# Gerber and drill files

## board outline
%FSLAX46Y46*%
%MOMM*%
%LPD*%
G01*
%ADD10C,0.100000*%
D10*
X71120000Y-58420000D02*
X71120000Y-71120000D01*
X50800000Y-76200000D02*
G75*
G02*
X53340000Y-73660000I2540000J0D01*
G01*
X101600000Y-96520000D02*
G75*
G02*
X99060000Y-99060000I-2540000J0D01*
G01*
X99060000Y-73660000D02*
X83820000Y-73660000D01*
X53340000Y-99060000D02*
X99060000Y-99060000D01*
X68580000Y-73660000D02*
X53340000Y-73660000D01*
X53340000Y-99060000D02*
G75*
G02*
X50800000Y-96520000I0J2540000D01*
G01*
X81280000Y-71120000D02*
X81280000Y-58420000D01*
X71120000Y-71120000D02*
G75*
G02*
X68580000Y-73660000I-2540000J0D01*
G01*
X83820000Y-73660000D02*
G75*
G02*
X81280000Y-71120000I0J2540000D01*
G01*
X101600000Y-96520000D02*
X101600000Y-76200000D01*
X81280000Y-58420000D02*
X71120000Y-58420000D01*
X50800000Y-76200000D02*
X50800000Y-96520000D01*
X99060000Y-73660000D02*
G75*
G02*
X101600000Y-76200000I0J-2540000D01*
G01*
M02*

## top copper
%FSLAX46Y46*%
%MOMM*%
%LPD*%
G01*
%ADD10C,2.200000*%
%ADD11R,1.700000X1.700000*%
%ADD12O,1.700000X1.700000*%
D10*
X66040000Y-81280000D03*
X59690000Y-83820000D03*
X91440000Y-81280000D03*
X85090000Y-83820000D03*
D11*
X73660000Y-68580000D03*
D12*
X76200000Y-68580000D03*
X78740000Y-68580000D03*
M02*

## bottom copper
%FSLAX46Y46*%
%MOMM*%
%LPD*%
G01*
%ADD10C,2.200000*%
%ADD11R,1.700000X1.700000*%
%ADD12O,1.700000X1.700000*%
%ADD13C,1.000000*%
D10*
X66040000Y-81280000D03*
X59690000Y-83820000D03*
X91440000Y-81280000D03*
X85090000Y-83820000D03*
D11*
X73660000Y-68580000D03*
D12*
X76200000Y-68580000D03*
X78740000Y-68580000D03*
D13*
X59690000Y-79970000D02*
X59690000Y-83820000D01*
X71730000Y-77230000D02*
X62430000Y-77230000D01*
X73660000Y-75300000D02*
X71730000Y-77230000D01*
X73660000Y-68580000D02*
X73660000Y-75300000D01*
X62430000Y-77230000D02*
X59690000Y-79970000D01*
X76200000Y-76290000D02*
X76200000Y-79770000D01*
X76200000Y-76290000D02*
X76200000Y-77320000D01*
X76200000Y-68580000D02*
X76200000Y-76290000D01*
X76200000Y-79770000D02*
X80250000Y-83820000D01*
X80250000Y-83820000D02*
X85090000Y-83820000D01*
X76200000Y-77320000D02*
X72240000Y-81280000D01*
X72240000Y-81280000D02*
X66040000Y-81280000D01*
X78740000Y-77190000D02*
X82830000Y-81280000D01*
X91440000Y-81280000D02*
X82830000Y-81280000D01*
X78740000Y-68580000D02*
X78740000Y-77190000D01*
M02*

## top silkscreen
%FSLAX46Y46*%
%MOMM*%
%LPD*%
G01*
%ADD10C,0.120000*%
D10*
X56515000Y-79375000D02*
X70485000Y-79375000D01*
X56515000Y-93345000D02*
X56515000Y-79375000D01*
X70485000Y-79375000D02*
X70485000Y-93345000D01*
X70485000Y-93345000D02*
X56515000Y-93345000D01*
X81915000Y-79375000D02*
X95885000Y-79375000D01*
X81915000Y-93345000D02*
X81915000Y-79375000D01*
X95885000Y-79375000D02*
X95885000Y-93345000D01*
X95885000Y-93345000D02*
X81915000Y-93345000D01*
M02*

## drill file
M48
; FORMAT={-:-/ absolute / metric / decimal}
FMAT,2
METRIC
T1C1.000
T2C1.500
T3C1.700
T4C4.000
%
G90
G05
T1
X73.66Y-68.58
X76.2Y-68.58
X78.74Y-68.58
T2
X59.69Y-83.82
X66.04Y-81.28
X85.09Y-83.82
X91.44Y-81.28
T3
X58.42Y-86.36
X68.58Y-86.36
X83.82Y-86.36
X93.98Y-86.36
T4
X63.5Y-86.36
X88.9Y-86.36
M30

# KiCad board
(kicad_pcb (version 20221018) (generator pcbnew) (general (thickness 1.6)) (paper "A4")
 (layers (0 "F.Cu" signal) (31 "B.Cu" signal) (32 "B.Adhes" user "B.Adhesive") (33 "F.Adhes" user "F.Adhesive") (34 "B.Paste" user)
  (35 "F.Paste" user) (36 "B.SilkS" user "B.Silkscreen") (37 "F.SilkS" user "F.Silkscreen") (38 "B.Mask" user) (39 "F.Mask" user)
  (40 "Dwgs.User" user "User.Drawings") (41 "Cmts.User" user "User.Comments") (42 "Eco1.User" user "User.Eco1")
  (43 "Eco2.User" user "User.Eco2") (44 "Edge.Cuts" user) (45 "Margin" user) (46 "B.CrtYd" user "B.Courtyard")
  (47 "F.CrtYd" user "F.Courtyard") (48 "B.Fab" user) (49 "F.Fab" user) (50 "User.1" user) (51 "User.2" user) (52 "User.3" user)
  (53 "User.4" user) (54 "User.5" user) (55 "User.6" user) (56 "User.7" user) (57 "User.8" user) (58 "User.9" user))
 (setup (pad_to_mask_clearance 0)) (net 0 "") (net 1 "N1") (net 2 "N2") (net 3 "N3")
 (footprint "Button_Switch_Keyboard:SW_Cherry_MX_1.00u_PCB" (layer "F.Cu") (at 66.04 81.28)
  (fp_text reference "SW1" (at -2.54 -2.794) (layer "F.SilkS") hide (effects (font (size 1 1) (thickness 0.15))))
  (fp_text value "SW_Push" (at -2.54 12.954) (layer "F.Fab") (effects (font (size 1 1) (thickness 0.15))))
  (fp_line (start -9.525 -1.905) (end 4.445 -1.905) (stroke (width 0.12) (type solid)) (layer "F.SilkS"))
  (fp_line (start -9.525 12.065) (end -9.525 -1.905) (stroke (width 0.12) (type solid)) (layer "F.SilkS"))
  (fp_line (start 4.445 -1.905) (end 4.445 12.065) (stroke (width 0.12) (type solid)) (layer "F.SilkS"))
  (fp_line (start 4.445 12.065) (end -9.525 12.065) (stroke (width 0.12) (type solid)) (layer "F.SilkS"))
  (pad "" np_thru_hole circle (at -7.62 5.08) (size 1.7 1.7) (drill 1.7) (layers "*.Cu" "*.Mask"))
  (pad "" np_thru_hole circle (at -2.54 5.08) (size 4 4) (drill 4) (layers "*.Cu" "*.Mask"))
  (pad "" np_thru_hole circle (at 2.54 5.08) (size 1.7 1.7) (drill 1.7) (layers "*.Cu" "*.Mask"))
  (pad "1" thru_hole circle (at 0 0) (size 2.2 2.2) (drill 1.5) (layers "*.Cu" "*.Mask") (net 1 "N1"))
  (pad "2" thru_hole circle (at -6.35 2.54) (size 2.2 2.2) (drill 1.5) (layers "*.Cu" "*.Mask") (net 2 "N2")))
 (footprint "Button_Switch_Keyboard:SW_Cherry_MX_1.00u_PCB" (layer "F.Cu") (at 91.44 81.28)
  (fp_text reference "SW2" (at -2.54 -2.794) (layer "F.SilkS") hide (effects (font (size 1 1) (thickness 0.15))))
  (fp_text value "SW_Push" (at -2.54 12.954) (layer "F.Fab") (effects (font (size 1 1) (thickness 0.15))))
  (fp_line (start -9.525 -1.905) (end 4.445 -1.905) (stroke (width 0.12) (type solid)) (layer "F.SilkS"))
  (fp_line (start -9.525 12.065) (end -9.525 -1.905) (stroke (width 0.12) (type solid)) (layer "F.SilkS"))
  (fp_line (start 4.445 -1.905) (end 4.445 12.065) (stroke (width 0.12) (type solid)) (layer "F.SilkS"))
  (fp_line (start 4.445 12.065) (end -9.525 12.065) (stroke (width 0.12) (type solid)) (layer "F.SilkS"))
  (pad "" np_thru_hole circle (at -7.62 5.08) (size 1.7 1.7) (drill 1.7) (layers "*.Cu" "*.Mask"))
  (pad "" np_thru_hole circle (at -2.54 5.08) (size 4 4) (drill 4) (layers "*.Cu" "*.Mask"))
  (pad "" np_thru_hole circle (at 2.54 5.08) (size 1.7 1.7) (drill 1.7) (layers "*.Cu" "*.Mask"))
  (pad "1" thru_hole circle (at 0 0) (size 2.2 2.2) (drill 1.5) (layers "*.Cu" "*.Mask") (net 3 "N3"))
  (pad "2" thru_hole circle (at -6.35 2.54) (size 2.2 2.2) (drill 1.5) (layers "*.Cu" "*.Mask") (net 1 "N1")))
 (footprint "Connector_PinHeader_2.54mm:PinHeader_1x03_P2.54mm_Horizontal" (layer "F.Cu") (at 73.66 68.58 90)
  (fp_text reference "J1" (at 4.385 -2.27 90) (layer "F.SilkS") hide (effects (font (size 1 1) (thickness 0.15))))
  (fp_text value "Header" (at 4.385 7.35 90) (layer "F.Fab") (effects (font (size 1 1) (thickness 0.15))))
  (pad "1" thru_hole rect (at 0 0 90) (size 1.7 1.7) (drill 1) (layers "*.Cu" "*.Mask") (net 2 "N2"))
  (pad "2" thru_hole oval (at 0 2.54 90) (size 1.7 1.7) (drill 1) (layers "*.Cu" "*.Mask") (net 1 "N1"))
  (pad "3" thru_hole oval (at 0 5.08 90) (size 1.7 1.7) (drill 1) (layers "*.Cu" "*.Mask") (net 3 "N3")))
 (gr_line (start 71.12 58.42) (end 71.12 71.12) (stroke (width 0.1) (type default)) (layer "Edge.Cuts"))
 (gr_arc (start 50.8 76.2) (mid 51.543949 74.403949) (end 53.34 73.66) (stroke (width 0.1) (type default)) (layer "Edge.Cuts"))
 (gr_arc (start 101.6 96.52) (mid 100.856051 98.316051) (end 99.06 99.06) (stroke (width 0.1) (type default)) (layer "Edge.Cuts"))
 (gr_line (start 99.06 73.66) (end 83.82 73.66) (stroke (width 0.1) (type default)) (layer "Edge.Cuts"))
 (gr_line (start 53.34 99.06) (end 99.06 99.06) (stroke (width 0.1) (type default)) (layer "Edge.Cuts"))
 (gr_line (start 68.58 73.66) (end 53.34 73.66) (stroke (width 0.1) (type default)) (layer "Edge.Cuts"))
 (gr_arc (start 53.34 99.06) (mid 51.543949 98.316051) (end 50.8 96.52) (stroke (width 0.1) (type default)) (layer "Edge.Cuts"))
 (gr_line (start 81.28 71.12) (end 81.28 58.42) (stroke (width 0.1) (type default)) (layer "Edge.Cuts"))
 (gr_arc (start 71.12 71.12) (mid 70.376051 72.916051) (end 68.58 73.66) (stroke (width 0.1) (type default)) (layer "Edge.Cuts"))
 (gr_arc (start 83.82 73.66) (mid 82.023949 72.916051) (end 81.28 71.12) (stroke (width 0.1) (type default)) (layer "Edge.Cuts"))
 (gr_line (start 101.6 96.52) (end 101.6 76.2) (stroke (width 0.1) (type default)) (layer "Edge.Cuts"))
 (gr_line (start 81.28 58.42) (end 71.12 58.42) (stroke (width 0.1) (type default)) (layer "Edge.Cuts"))
 (gr_line (start 50.8 76.2) (end 50.8 96.52) (stroke (width 0.1) (type default)) (layer "Edge.Cuts"))
 (gr_arc (start 99.06 73.66) (mid 100.856051 74.403949) (end 101.6 76.2) (stroke (width 0.1) (type default)) (layer "Edge.Cuts"))
 (segment (start 59.69 79.97) (end 59.69 83.82) (width 1) (layer "B.Cu") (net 2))
 (segment (start 71.73 77.23) (end 62.43 77.23) (width 1) (layer "B.Cu") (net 2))
 (segment (start 73.66 75.3) (end 71.73 77.23) (width 1) (layer "B.Cu") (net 2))
 (segment (start 73.66 68.58) (end 73.66 75.3) (width 1) (layer "B.Cu") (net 2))
 (segment (start 62.43 77.23) (end 59.69 79.97) (width 1) (layer "B.Cu") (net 2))
 (segment (start 76.2 76.29) (end 76.2 79.77) (width 1) (layer "B.Cu") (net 1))
 (segment (start 76.2 76.29) (end 76.2 77.32) (width 1) (layer "B.Cu") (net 1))
 (segment (start 76.2 68.58) (end 76.2 76.29) (width 1) (layer "B.Cu") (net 1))
 (segment (start 76.2 79.77) (end 80.25 83.82) (width 1) (layer "B.Cu") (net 1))
 (segment (start 80.25 83.82) (end 85.09 83.82) (width 1) (layer "B.Cu") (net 1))
 (segment (start 76.2 77.32) (end 72.24 81.28) (width 1) (layer "B.Cu") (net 1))
 (segment (start 72.24 81.28) (end 66.04 81.28) (width 1) (layer "B.Cu") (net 1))
 (segment (start 78.74 77.19) (end 82.83 81.28) (width 1) (layer "B.Cu") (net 3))
 (segment (start 91.44 81.28) (end 82.83 81.28) (width 1) (layer "B.Cu") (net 3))
 (segment (start 78.74 68.58) (end 78.74 77.19) (width 1) (layer "B.Cu") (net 3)))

